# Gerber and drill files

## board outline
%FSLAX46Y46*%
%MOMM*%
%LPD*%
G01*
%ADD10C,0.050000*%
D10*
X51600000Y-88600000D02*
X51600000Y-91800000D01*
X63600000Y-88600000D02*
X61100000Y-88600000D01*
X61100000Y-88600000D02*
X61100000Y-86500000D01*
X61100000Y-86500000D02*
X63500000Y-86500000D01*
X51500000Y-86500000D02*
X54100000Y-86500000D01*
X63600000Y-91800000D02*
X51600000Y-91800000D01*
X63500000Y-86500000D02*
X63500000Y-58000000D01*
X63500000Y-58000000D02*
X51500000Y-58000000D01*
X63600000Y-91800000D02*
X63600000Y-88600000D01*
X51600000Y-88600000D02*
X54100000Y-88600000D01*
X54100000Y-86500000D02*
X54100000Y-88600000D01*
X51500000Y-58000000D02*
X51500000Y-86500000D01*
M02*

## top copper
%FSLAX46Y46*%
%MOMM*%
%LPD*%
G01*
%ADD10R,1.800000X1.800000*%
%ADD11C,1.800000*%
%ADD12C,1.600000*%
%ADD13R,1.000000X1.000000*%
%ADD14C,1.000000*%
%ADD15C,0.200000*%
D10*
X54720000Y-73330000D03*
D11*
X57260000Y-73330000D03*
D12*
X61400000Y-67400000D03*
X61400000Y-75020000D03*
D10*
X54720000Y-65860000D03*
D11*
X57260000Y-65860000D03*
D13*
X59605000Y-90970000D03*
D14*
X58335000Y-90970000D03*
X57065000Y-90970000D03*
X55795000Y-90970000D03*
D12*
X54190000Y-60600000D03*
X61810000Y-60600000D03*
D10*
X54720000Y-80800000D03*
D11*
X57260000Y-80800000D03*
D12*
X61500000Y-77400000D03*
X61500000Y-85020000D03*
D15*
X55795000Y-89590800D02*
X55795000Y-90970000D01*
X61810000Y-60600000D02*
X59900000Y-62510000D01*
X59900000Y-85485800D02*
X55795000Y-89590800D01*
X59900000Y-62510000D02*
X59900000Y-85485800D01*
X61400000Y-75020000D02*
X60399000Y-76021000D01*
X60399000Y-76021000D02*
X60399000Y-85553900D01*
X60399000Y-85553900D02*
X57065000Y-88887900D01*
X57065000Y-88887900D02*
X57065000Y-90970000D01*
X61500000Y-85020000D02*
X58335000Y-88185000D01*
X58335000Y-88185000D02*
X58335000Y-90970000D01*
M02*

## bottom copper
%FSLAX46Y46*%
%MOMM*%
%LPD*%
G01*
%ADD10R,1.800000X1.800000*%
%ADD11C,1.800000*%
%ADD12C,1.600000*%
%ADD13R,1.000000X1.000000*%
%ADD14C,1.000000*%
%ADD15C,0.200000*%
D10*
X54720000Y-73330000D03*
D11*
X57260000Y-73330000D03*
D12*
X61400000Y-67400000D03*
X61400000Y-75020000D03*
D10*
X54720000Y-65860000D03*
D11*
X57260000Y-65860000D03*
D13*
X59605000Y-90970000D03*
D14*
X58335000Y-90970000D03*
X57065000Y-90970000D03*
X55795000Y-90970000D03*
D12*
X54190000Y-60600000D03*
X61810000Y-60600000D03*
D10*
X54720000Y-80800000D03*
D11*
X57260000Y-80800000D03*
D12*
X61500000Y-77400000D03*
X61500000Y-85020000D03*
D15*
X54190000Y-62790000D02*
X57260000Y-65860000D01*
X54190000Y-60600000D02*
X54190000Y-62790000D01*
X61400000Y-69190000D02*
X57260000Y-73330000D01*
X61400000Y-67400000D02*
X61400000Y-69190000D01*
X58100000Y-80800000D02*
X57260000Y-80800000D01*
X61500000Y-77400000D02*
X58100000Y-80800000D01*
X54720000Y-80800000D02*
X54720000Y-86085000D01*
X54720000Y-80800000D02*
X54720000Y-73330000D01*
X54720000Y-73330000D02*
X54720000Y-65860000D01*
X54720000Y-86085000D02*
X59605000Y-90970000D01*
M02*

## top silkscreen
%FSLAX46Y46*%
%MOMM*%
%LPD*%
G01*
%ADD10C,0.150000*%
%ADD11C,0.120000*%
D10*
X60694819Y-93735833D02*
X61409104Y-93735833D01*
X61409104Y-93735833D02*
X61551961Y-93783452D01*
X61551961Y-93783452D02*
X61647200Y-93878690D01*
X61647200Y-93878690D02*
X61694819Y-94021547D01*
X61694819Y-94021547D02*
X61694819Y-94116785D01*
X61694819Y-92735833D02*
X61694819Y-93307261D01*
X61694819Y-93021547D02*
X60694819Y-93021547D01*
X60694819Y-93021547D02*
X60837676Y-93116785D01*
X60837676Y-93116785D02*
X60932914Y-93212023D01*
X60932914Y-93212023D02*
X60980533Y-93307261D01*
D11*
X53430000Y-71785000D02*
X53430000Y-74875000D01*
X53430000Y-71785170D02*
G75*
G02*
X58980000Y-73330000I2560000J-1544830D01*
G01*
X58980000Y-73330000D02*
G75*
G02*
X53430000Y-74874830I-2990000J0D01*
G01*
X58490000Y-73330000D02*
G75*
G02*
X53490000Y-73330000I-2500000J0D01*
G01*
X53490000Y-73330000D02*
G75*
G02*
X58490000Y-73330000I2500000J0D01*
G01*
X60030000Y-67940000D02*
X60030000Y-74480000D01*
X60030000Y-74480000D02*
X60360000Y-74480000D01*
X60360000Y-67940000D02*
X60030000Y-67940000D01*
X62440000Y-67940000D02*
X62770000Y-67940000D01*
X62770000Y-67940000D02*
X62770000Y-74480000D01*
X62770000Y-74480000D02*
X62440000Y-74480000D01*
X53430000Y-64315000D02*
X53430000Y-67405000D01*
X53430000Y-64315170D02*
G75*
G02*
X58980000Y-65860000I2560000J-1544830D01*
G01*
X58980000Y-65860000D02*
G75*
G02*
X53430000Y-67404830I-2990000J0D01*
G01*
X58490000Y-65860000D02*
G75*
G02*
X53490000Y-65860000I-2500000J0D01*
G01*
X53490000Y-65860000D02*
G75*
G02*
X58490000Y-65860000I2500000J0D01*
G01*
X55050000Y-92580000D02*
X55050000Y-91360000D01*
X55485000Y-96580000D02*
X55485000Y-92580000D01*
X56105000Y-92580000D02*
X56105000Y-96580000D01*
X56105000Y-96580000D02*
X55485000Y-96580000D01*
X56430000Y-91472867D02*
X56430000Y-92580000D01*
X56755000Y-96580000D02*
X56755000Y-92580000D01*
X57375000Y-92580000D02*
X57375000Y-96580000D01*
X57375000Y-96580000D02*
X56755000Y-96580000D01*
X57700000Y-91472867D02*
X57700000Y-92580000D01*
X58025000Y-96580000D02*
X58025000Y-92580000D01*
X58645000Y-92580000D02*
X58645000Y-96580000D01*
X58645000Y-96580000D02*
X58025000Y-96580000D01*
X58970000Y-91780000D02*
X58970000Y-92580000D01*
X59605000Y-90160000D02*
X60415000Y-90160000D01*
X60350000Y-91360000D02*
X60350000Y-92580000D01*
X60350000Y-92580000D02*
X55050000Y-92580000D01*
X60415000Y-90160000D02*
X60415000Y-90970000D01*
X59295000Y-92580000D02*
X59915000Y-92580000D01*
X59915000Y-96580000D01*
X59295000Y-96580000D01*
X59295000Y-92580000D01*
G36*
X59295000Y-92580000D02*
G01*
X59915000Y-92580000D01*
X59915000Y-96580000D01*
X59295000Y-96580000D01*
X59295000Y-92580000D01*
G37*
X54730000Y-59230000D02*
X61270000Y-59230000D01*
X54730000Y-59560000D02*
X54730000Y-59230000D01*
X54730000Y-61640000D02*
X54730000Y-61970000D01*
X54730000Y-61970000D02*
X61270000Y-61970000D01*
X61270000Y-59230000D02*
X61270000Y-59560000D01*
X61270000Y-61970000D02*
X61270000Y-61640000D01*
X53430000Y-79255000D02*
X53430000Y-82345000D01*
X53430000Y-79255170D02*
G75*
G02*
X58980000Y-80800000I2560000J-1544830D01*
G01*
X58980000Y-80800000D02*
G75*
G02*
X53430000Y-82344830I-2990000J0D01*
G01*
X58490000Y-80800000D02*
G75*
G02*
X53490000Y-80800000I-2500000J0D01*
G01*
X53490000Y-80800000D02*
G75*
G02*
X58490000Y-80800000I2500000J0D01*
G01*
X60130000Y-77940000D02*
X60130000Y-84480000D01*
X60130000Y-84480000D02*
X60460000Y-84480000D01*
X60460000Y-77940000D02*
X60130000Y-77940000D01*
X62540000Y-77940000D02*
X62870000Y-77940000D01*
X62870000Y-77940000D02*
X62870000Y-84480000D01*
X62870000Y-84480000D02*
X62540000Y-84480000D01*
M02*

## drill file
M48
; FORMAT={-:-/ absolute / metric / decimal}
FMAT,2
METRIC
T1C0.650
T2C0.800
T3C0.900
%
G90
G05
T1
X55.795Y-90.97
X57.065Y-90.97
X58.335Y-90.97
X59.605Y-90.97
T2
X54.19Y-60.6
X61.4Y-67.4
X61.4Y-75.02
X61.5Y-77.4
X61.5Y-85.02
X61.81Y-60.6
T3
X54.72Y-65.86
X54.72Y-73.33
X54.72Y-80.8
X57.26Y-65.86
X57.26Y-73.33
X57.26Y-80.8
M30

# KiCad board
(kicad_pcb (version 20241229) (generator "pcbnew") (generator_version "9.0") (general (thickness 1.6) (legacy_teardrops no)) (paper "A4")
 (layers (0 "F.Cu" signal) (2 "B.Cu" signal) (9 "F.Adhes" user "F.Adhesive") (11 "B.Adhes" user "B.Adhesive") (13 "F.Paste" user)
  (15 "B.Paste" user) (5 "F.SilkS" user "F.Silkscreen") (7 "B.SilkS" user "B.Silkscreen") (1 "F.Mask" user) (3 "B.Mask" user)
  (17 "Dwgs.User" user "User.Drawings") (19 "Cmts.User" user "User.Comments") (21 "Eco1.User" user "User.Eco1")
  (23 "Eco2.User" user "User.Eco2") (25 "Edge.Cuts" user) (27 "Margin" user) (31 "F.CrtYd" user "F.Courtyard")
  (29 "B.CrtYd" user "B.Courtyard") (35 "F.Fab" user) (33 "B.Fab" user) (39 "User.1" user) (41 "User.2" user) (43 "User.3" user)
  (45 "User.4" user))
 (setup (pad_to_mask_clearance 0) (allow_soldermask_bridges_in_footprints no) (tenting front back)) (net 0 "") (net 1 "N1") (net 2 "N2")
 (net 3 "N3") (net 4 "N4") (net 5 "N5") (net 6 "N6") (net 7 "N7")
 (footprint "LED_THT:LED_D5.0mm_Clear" (layer "F.Cu") (at 54.72 73.33)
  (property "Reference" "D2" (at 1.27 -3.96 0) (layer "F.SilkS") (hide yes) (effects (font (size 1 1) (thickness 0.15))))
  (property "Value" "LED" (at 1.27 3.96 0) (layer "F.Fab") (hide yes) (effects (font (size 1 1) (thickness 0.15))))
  (fp_line (start -1.29 -1.545) (end -1.29 1.545) (stroke (width 0.12) (type solid)) (layer "F.SilkS"))
  (fp_arc (start -1.29 -1.54483) (mid 2.071779 -2.880495) (end 4.26 0) (stroke (width 0.12) (type solid)) (layer "F.SilkS"))
  (fp_arc (start 4.26 0) (mid 2.071779 2.880495) (end -1.29 1.54483) (stroke (width 0.12) (type solid)) (layer "F.SilkS"))
  (fp_circle (center 1.27 0) (end 3.77 0) (stroke (width 0.12) (type solid)) (fill no) (layer "F.SilkS"))
  (pad "1" thru_hole rect (at 0 0) (size 1.8 1.8) (drill 0.9) (layers "*.Cu" "*.Mask") (remove_unused_layers no) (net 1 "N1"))
  (pad "2" thru_hole circle (at 2.54 0) (size 1.8 1.8) (drill 0.9) (layers "*.Cu" "*.Mask") (remove_unused_layers no) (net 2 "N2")))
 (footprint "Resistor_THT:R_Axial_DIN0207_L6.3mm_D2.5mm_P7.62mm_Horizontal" (layer "F.Cu") (at 61.4 67.4 -90)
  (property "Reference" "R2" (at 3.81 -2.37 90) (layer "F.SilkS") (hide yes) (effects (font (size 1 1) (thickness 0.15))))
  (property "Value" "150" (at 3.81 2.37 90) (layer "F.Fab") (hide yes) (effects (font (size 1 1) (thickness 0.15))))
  (fp_line (start 0.54 1.37) (end 7.08 1.37) (stroke (width 0.12) (type solid)) (layer "F.SilkS"))
  (fp_line (start 7.08 1.37) (end 7.08 1.04) (stroke (width 0.12) (type solid)) (layer "F.SilkS"))
  (fp_line (start 0.54 1.04) (end 0.54 1.37) (stroke (width 0.12) (type solid)) (layer "F.SilkS"))
  (fp_line (start 0.54 -1.04) (end 0.54 -1.37) (stroke (width 0.12) (type solid)) (layer "F.SilkS"))
  (fp_line (start 0.54 -1.37) (end 7.08 -1.37) (stroke (width 0.12) (type solid)) (layer "F.SilkS"))
  (fp_line (start 7.08 -1.37) (end 7.08 -1.04) (stroke (width 0.12) (type solid)) (layer "F.SilkS"))
  (pad "1" thru_hole circle (at 0 0 270) (size 1.6 1.6) (drill 0.8) (layers "*.Cu" "*.Mask") (remove_unused_layers no) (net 2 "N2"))
  (pad "2" thru_hole circle (at 7.62 0 270) (size 1.6 1.6) (drill 0.8) (layers "*.Cu" "*.Mask") (remove_unused_layers no) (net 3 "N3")))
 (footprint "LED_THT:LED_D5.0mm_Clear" (layer "F.Cu") (at 54.72 65.86)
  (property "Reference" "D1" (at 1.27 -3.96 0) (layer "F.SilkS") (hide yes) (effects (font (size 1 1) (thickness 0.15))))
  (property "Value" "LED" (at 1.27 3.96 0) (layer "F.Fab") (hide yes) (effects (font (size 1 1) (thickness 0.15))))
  (fp_line (start -1.29 -1.545) (end -1.29 1.545) (stroke (width 0.12) (type solid)) (layer "F.SilkS"))
  (fp_arc (start -1.29 -1.54483) (mid 2.071779 -2.880495) (end 4.26 0) (stroke (width 0.12) (type solid)) (layer "F.SilkS"))
  (fp_arc (start 4.26 0) (mid 2.071779 2.880495) (end -1.29 1.54483) (stroke (width 0.12) (type solid)) (layer "F.SilkS"))
  (fp_circle (center 1.27 0) (end 3.77 0) (stroke (width 0.12) (type solid)) (fill no) (layer "F.SilkS"))
  (pad "1" thru_hole rect (at 0 0) (size 1.8 1.8) (drill 0.9) (layers "*.Cu" "*.Mask") (remove_unused_layers no) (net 1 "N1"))
  (pad "2" thru_hole circle (at 2.54 0) (size 1.8 1.8) (drill 0.9) (layers "*.Cu" "*.Mask") (remove_unused_layers no) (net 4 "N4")))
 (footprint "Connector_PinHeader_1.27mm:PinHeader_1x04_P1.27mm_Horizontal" (layer "F.Cu") (at 59.605 90.97 -90)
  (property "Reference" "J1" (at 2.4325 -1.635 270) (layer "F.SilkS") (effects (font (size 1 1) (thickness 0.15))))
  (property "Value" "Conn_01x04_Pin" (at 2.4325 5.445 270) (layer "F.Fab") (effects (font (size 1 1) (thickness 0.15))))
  (fp_line (start 1.61 4.555) (end 0.39 4.555) (stroke (width 0.12) (type solid)) (layer "F.SilkS"))
  (fp_line (start 5.61 4.12) (end 1.61 4.12) (stroke (width 0.12) (type solid)) (layer "F.SilkS"))
  (fp_line (start 1.61 3.5) (end 5.61 3.5) (stroke (width 0.12) (type solid)) (layer "F.SilkS"))
  (fp_line (start 5.61 3.5) (end 5.61 4.12) (stroke (width 0.12) (type solid)) (layer "F.SilkS"))
  (fp_line (start 0.502867 3.175) (end 1.61 3.175) (stroke (width 0.12) (type solid)) (layer "F.SilkS"))
  (fp_line (start 5.61 2.85) (end 1.61 2.85) (stroke (width 0.12) (type solid)) (layer "F.SilkS"))
  (fp_line (start 1.61 2.23) (end 5.61 2.23) (stroke (width 0.12) (type solid)) (layer "F.SilkS"))
  (fp_line (start 5.61 2.23) (end 5.61 2.85) (stroke (width 0.12) (type solid)) (layer "F.SilkS"))
  (fp_line (start 0.502867 1.905) (end 1.61 1.905) (stroke (width 0.12) (type solid)) (layer "F.SilkS"))
  (fp_line (start 5.61 1.58) (end 1.61 1.58) (stroke (width 0.12) (type solid)) (layer "F.SilkS"))
  (fp_line (start 1.61 0.96) (end 5.61 0.96) (stroke (width 0.12) (type solid)) (layer "F.SilkS"))
  (fp_line (start 5.61 0.96) (end 5.61 1.58) (stroke (width 0.12) (type solid)) (layer "F.SilkS"))
  (fp_line (start 0.81 0.635) (end 1.61 0.635) (stroke (width 0.12) (type solid)) (layer "F.SilkS"))
  (fp_line (start -0.81 0) (end -0.81 -0.81) (stroke (width 0.12) (type solid)) (layer "F.SilkS"))
  (fp_line (start 0.39 -0.745) (end 1.61 -0.745) (stroke (width 0.12) (type solid)) (layer "F.SilkS"))
  (fp_line (start 1.61 -0.745) (end 1.61 4.555) (stroke (width 0.12) (type solid)) (layer "F.SilkS"))
  (fp_line (start -0.81 -0.81) (end 0 -0.81) (stroke (width 0.12) (type solid)) (layer "F.SilkS"))
  (fp_rect (start 1.61 -0.31) (end 5.61 0.31) (stroke (width 0.12) (type solid)) (fill yes) (layer "F.SilkS"))
  (pad "1" thru_hole rect (at 0 0 270) (size 1 1) (drill 0.65) (layers "*.Cu" "*.Mask") (remove_unused_layers no) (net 1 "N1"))
  (pad "2" thru_hole circle (at 0 1.27 270) (size 1 1) (drill 0.65) (layers "*.Cu" "*.Mask") (remove_unused_layers no) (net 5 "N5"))
  (pad "3" thru_hole circle (at 0 2.54 270) (size 1 1) (drill 0.65) (layers "*.Cu" "*.Mask") (remove_unused_layers no) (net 3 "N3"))
  (pad "4" thru_hole circle (at 0 3.81 270) (size 1 1) (drill 0.65) (layers "*.Cu" "*.Mask") (remove_unused_layers no) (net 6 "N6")))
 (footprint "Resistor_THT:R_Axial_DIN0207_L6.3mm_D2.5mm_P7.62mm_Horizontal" (layer "F.Cu") (at 54.19 60.6)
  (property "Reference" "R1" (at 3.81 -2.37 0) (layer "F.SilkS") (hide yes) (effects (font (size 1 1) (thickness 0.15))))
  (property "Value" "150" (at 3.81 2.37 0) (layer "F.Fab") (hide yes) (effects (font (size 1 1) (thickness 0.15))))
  (fp_line (start 0.54 -1.37) (end 7.08 -1.37) (stroke (width 0.12) (type solid)) (layer "F.SilkS"))
  (fp_line (start 0.54 -1.04) (end 0.54 -1.37) (stroke (width 0.12) (type solid)) (layer "F.SilkS"))
  (fp_line (start 0.54 1.04) (end 0.54 1.37) (stroke (width 0.12) (type solid)) (layer "F.SilkS"))
  (fp_line (start 0.54 1.37) (end 7.08 1.37) (stroke (width 0.12) (type solid)) (layer "F.SilkS"))
  (fp_line (start 7.08 -1.37) (end 7.08 -1.04) (stroke (width 0.12) (type solid)) (layer "F.SilkS"))
  (fp_line (start 7.08 1.37) (end 7.08 1.04) (stroke (width 0.12) (type solid)) (layer "F.SilkS"))
  (pad "1" thru_hole circle (at 0 0) (size 1.6 1.6) (drill 0.8) (layers "*.Cu" "*.Mask") (remove_unused_layers no) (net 4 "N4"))
  (pad "2" thru_hole circle (at 7.62 0) (size 1.6 1.6) (drill 0.8) (layers "*.Cu" "*.Mask") (remove_unused_layers no) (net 6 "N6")))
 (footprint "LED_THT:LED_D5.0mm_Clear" (layer "F.Cu") (at 54.72 80.8)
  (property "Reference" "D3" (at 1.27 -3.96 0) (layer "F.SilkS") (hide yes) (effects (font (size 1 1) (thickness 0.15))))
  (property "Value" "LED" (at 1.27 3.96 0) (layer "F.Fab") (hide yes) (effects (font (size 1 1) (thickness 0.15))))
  (fp_line (start -1.29 -1.545) (end -1.29 1.545) (stroke (width 0.12) (type solid)) (layer "F.SilkS"))
  (fp_arc (start -1.29 -1.54483) (mid 2.071779 -2.880495) (end 4.26 0) (stroke (width 0.12) (type solid)) (layer "F.SilkS"))
  (fp_arc (start 4.26 0) (mid 2.071779 2.880495) (end -1.29 1.54483) (stroke (width 0.12) (type solid)) (layer "F.SilkS"))
  (fp_circle (center 1.27 0) (end 3.77 0) (stroke (width 0.12) (type solid)) (fill no) (layer "F.SilkS"))
  (pad "1" thru_hole rect (at 0 0) (size 1.8 1.8) (drill 0.9) (layers "*.Cu" "*.Mask") (remove_unused_layers no) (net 1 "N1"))
  (pad "2" thru_hole circle (at 2.54 0) (size 1.8 1.8) (drill 0.9) (layers "*.Cu" "*.Mask") (remove_unused_layers no) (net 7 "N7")))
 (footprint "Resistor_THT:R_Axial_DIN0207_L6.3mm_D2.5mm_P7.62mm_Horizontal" (layer "F.Cu") (at 61.5 77.4 -90)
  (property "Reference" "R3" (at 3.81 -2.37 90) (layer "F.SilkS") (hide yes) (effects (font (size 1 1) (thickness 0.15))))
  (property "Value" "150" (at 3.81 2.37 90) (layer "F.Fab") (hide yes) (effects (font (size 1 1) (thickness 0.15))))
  (fp_line (start 0.54 1.37) (end 7.08 1.37) (stroke (width 0.12) (type solid)) (layer "F.SilkS"))
  (fp_line (start 7.08 1.37) (end 7.08 1.04) (stroke (width 0.12) (type solid)) (layer "F.SilkS"))
  (fp_line (start 0.54 1.04) (end 0.54 1.37) (stroke (width 0.12) (type solid)) (layer "F.SilkS"))
  (fp_line (start 0.54 -1.04) (end 0.54 -1.37) (stroke (width 0.12) (type solid)) (layer "F.SilkS"))
  (fp_line (start 0.54 -1.37) (end 7.08 -1.37) (stroke (width 0.12) (type solid)) (layer "F.SilkS"))
  (fp_line (start 7.08 -1.37) (end 7.08 -1.04) (stroke (width 0.12) (type solid)) (layer "F.SilkS"))
  (pad "1" thru_hole circle (at 0 0 270) (size 1.6 1.6) (drill 0.8) (layers "*.Cu" "*.Mask") (remove_unused_layers no) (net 7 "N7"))
  (pad "2" thru_hole circle (at 7.62 0 270) (size 1.6 1.6) (drill 0.8) (layers "*.Cu" "*.Mask") (remove_unused_layers no) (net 5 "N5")))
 (gr_line (start 51.6 88.6) (end 51.6 91.8) (stroke (width 0.05) (type default)) (layer "Edge.Cuts"))
 (gr_line (start 63.6 88.6) (end 61.1 88.6) (stroke (width 0.05) (type default)) (layer "Edge.Cuts"))
 (gr_line (start 61.1 88.6) (end 61.1 86.5) (stroke (width 0.05) (type default)) (layer "Edge.Cuts"))
 (gr_line (start 61.1 86.5) (end 63.5 86.5) (stroke (width 0.05) (type default)) (layer "Edge.Cuts"))
 (gr_line (start 51.5 86.5) (end 54.1 86.5) (stroke (width 0.05) (type default)) (layer "Edge.Cuts"))
 (gr_line (start 63.6 91.8) (end 51.6 91.8) (stroke (width 0.05) (type default)) (layer "Edge.Cuts"))
 (gr_line (start 63.5 86.5) (end 63.5 58) (stroke (width 0.05) (type default)) (layer "Edge.Cuts"))
 (gr_line (start 63.5 58) (end 51.5 58) (stroke (width 0.05) (type default)) (layer "Edge.Cuts"))
 (gr_line (start 63.6 91.8) (end 63.6 88.6) (stroke (width 0.05) (type default)) (layer "Edge.Cuts"))
 (gr_line (start 51.6 88.6) (end 54.1 88.6) (stroke (width 0.05) (type default)) (layer "Edge.Cuts"))
 (gr_line (start 54.1 86.5) (end 54.1 88.6) (stroke (width 0.05) (type default)) (layer "Edge.Cuts"))
 (gr_line (start 51.5 58) (end 51.5 86.5) (stroke (width 0.05) (type default)) (layer "Edge.Cuts"))
 (segment (start 54.19 62.79) (end 57.26 65.86) (width 0.2) (layer "B.Cu") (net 4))
 (segment (start 54.19 60.6) (end 54.19 62.79) (width 0.2) (layer "B.Cu") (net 4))
 (segment (start 61.4 69.19) (end 57.26 73.33) (width 0.2) (layer "B.Cu") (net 2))
 (segment (start 61.4 67.4) (end 61.4 69.19) (width 0.2) (layer "B.Cu") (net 2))
 (segment (start 58.1 80.8) (end 57.26 80.8) (width 0.2) (layer "B.Cu") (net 7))
 (segment (start 61.5 77.4) (end 58.1 80.8) (width 0.2) (layer "B.Cu") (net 7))
 (segment (start 54.72 80.8) (end 54.72 86.085) (width 0.2) (layer "B.Cu") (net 1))
 (segment (start 54.72 80.8) (end 54.72 73.33) (width 0.2) (layer "B.Cu") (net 1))
 (segment (start 54.72 73.33) (end 54.72 65.86) (width 0.2) (layer "B.Cu") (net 1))
 (segment (start 54.72 86.085) (end 59.605 90.97) (width 0.2) (layer "B.Cu") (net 1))
 (segment (start 55.795 89.5908) (end 55.795 90.97) (width 0.2) (layer "F.Cu") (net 6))
 (segment (start 61.81 60.6) (end 59.9 62.51) (width 0.2) (layer "F.Cu") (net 6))
 (segment (start 59.9 85.4858) (end 55.795 89.5908) (width 0.2) (layer "F.Cu") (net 6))
 (segment (start 59.9 62.51) (end 59.9 85.4858) (width 0.2) (layer "F.Cu") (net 6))
 (segment (start 61.4 75.02) (end 60.399 76.021) (width 0.2) (layer "F.Cu") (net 3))
 (segment (start 60.399 76.021) (end 60.399 85.5539) (width 0.2) (layer "F.Cu") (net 3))
 (segment (start 60.399 85.5539) (end 57.065 88.8879) (width 0.2) (layer "F.Cu") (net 3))
 (segment (start 57.065 88.8879) (end 57.065 90.97) (width 0.2) (layer "F.Cu") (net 3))
 (segment (start 61.5 85.02) (end 58.335 88.185) (width 0.2) (layer "F.Cu") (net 5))
 (segment (start 58.335 88.185) (end 58.335 90.97) (width 0.2) (layer "F.Cu") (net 5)))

